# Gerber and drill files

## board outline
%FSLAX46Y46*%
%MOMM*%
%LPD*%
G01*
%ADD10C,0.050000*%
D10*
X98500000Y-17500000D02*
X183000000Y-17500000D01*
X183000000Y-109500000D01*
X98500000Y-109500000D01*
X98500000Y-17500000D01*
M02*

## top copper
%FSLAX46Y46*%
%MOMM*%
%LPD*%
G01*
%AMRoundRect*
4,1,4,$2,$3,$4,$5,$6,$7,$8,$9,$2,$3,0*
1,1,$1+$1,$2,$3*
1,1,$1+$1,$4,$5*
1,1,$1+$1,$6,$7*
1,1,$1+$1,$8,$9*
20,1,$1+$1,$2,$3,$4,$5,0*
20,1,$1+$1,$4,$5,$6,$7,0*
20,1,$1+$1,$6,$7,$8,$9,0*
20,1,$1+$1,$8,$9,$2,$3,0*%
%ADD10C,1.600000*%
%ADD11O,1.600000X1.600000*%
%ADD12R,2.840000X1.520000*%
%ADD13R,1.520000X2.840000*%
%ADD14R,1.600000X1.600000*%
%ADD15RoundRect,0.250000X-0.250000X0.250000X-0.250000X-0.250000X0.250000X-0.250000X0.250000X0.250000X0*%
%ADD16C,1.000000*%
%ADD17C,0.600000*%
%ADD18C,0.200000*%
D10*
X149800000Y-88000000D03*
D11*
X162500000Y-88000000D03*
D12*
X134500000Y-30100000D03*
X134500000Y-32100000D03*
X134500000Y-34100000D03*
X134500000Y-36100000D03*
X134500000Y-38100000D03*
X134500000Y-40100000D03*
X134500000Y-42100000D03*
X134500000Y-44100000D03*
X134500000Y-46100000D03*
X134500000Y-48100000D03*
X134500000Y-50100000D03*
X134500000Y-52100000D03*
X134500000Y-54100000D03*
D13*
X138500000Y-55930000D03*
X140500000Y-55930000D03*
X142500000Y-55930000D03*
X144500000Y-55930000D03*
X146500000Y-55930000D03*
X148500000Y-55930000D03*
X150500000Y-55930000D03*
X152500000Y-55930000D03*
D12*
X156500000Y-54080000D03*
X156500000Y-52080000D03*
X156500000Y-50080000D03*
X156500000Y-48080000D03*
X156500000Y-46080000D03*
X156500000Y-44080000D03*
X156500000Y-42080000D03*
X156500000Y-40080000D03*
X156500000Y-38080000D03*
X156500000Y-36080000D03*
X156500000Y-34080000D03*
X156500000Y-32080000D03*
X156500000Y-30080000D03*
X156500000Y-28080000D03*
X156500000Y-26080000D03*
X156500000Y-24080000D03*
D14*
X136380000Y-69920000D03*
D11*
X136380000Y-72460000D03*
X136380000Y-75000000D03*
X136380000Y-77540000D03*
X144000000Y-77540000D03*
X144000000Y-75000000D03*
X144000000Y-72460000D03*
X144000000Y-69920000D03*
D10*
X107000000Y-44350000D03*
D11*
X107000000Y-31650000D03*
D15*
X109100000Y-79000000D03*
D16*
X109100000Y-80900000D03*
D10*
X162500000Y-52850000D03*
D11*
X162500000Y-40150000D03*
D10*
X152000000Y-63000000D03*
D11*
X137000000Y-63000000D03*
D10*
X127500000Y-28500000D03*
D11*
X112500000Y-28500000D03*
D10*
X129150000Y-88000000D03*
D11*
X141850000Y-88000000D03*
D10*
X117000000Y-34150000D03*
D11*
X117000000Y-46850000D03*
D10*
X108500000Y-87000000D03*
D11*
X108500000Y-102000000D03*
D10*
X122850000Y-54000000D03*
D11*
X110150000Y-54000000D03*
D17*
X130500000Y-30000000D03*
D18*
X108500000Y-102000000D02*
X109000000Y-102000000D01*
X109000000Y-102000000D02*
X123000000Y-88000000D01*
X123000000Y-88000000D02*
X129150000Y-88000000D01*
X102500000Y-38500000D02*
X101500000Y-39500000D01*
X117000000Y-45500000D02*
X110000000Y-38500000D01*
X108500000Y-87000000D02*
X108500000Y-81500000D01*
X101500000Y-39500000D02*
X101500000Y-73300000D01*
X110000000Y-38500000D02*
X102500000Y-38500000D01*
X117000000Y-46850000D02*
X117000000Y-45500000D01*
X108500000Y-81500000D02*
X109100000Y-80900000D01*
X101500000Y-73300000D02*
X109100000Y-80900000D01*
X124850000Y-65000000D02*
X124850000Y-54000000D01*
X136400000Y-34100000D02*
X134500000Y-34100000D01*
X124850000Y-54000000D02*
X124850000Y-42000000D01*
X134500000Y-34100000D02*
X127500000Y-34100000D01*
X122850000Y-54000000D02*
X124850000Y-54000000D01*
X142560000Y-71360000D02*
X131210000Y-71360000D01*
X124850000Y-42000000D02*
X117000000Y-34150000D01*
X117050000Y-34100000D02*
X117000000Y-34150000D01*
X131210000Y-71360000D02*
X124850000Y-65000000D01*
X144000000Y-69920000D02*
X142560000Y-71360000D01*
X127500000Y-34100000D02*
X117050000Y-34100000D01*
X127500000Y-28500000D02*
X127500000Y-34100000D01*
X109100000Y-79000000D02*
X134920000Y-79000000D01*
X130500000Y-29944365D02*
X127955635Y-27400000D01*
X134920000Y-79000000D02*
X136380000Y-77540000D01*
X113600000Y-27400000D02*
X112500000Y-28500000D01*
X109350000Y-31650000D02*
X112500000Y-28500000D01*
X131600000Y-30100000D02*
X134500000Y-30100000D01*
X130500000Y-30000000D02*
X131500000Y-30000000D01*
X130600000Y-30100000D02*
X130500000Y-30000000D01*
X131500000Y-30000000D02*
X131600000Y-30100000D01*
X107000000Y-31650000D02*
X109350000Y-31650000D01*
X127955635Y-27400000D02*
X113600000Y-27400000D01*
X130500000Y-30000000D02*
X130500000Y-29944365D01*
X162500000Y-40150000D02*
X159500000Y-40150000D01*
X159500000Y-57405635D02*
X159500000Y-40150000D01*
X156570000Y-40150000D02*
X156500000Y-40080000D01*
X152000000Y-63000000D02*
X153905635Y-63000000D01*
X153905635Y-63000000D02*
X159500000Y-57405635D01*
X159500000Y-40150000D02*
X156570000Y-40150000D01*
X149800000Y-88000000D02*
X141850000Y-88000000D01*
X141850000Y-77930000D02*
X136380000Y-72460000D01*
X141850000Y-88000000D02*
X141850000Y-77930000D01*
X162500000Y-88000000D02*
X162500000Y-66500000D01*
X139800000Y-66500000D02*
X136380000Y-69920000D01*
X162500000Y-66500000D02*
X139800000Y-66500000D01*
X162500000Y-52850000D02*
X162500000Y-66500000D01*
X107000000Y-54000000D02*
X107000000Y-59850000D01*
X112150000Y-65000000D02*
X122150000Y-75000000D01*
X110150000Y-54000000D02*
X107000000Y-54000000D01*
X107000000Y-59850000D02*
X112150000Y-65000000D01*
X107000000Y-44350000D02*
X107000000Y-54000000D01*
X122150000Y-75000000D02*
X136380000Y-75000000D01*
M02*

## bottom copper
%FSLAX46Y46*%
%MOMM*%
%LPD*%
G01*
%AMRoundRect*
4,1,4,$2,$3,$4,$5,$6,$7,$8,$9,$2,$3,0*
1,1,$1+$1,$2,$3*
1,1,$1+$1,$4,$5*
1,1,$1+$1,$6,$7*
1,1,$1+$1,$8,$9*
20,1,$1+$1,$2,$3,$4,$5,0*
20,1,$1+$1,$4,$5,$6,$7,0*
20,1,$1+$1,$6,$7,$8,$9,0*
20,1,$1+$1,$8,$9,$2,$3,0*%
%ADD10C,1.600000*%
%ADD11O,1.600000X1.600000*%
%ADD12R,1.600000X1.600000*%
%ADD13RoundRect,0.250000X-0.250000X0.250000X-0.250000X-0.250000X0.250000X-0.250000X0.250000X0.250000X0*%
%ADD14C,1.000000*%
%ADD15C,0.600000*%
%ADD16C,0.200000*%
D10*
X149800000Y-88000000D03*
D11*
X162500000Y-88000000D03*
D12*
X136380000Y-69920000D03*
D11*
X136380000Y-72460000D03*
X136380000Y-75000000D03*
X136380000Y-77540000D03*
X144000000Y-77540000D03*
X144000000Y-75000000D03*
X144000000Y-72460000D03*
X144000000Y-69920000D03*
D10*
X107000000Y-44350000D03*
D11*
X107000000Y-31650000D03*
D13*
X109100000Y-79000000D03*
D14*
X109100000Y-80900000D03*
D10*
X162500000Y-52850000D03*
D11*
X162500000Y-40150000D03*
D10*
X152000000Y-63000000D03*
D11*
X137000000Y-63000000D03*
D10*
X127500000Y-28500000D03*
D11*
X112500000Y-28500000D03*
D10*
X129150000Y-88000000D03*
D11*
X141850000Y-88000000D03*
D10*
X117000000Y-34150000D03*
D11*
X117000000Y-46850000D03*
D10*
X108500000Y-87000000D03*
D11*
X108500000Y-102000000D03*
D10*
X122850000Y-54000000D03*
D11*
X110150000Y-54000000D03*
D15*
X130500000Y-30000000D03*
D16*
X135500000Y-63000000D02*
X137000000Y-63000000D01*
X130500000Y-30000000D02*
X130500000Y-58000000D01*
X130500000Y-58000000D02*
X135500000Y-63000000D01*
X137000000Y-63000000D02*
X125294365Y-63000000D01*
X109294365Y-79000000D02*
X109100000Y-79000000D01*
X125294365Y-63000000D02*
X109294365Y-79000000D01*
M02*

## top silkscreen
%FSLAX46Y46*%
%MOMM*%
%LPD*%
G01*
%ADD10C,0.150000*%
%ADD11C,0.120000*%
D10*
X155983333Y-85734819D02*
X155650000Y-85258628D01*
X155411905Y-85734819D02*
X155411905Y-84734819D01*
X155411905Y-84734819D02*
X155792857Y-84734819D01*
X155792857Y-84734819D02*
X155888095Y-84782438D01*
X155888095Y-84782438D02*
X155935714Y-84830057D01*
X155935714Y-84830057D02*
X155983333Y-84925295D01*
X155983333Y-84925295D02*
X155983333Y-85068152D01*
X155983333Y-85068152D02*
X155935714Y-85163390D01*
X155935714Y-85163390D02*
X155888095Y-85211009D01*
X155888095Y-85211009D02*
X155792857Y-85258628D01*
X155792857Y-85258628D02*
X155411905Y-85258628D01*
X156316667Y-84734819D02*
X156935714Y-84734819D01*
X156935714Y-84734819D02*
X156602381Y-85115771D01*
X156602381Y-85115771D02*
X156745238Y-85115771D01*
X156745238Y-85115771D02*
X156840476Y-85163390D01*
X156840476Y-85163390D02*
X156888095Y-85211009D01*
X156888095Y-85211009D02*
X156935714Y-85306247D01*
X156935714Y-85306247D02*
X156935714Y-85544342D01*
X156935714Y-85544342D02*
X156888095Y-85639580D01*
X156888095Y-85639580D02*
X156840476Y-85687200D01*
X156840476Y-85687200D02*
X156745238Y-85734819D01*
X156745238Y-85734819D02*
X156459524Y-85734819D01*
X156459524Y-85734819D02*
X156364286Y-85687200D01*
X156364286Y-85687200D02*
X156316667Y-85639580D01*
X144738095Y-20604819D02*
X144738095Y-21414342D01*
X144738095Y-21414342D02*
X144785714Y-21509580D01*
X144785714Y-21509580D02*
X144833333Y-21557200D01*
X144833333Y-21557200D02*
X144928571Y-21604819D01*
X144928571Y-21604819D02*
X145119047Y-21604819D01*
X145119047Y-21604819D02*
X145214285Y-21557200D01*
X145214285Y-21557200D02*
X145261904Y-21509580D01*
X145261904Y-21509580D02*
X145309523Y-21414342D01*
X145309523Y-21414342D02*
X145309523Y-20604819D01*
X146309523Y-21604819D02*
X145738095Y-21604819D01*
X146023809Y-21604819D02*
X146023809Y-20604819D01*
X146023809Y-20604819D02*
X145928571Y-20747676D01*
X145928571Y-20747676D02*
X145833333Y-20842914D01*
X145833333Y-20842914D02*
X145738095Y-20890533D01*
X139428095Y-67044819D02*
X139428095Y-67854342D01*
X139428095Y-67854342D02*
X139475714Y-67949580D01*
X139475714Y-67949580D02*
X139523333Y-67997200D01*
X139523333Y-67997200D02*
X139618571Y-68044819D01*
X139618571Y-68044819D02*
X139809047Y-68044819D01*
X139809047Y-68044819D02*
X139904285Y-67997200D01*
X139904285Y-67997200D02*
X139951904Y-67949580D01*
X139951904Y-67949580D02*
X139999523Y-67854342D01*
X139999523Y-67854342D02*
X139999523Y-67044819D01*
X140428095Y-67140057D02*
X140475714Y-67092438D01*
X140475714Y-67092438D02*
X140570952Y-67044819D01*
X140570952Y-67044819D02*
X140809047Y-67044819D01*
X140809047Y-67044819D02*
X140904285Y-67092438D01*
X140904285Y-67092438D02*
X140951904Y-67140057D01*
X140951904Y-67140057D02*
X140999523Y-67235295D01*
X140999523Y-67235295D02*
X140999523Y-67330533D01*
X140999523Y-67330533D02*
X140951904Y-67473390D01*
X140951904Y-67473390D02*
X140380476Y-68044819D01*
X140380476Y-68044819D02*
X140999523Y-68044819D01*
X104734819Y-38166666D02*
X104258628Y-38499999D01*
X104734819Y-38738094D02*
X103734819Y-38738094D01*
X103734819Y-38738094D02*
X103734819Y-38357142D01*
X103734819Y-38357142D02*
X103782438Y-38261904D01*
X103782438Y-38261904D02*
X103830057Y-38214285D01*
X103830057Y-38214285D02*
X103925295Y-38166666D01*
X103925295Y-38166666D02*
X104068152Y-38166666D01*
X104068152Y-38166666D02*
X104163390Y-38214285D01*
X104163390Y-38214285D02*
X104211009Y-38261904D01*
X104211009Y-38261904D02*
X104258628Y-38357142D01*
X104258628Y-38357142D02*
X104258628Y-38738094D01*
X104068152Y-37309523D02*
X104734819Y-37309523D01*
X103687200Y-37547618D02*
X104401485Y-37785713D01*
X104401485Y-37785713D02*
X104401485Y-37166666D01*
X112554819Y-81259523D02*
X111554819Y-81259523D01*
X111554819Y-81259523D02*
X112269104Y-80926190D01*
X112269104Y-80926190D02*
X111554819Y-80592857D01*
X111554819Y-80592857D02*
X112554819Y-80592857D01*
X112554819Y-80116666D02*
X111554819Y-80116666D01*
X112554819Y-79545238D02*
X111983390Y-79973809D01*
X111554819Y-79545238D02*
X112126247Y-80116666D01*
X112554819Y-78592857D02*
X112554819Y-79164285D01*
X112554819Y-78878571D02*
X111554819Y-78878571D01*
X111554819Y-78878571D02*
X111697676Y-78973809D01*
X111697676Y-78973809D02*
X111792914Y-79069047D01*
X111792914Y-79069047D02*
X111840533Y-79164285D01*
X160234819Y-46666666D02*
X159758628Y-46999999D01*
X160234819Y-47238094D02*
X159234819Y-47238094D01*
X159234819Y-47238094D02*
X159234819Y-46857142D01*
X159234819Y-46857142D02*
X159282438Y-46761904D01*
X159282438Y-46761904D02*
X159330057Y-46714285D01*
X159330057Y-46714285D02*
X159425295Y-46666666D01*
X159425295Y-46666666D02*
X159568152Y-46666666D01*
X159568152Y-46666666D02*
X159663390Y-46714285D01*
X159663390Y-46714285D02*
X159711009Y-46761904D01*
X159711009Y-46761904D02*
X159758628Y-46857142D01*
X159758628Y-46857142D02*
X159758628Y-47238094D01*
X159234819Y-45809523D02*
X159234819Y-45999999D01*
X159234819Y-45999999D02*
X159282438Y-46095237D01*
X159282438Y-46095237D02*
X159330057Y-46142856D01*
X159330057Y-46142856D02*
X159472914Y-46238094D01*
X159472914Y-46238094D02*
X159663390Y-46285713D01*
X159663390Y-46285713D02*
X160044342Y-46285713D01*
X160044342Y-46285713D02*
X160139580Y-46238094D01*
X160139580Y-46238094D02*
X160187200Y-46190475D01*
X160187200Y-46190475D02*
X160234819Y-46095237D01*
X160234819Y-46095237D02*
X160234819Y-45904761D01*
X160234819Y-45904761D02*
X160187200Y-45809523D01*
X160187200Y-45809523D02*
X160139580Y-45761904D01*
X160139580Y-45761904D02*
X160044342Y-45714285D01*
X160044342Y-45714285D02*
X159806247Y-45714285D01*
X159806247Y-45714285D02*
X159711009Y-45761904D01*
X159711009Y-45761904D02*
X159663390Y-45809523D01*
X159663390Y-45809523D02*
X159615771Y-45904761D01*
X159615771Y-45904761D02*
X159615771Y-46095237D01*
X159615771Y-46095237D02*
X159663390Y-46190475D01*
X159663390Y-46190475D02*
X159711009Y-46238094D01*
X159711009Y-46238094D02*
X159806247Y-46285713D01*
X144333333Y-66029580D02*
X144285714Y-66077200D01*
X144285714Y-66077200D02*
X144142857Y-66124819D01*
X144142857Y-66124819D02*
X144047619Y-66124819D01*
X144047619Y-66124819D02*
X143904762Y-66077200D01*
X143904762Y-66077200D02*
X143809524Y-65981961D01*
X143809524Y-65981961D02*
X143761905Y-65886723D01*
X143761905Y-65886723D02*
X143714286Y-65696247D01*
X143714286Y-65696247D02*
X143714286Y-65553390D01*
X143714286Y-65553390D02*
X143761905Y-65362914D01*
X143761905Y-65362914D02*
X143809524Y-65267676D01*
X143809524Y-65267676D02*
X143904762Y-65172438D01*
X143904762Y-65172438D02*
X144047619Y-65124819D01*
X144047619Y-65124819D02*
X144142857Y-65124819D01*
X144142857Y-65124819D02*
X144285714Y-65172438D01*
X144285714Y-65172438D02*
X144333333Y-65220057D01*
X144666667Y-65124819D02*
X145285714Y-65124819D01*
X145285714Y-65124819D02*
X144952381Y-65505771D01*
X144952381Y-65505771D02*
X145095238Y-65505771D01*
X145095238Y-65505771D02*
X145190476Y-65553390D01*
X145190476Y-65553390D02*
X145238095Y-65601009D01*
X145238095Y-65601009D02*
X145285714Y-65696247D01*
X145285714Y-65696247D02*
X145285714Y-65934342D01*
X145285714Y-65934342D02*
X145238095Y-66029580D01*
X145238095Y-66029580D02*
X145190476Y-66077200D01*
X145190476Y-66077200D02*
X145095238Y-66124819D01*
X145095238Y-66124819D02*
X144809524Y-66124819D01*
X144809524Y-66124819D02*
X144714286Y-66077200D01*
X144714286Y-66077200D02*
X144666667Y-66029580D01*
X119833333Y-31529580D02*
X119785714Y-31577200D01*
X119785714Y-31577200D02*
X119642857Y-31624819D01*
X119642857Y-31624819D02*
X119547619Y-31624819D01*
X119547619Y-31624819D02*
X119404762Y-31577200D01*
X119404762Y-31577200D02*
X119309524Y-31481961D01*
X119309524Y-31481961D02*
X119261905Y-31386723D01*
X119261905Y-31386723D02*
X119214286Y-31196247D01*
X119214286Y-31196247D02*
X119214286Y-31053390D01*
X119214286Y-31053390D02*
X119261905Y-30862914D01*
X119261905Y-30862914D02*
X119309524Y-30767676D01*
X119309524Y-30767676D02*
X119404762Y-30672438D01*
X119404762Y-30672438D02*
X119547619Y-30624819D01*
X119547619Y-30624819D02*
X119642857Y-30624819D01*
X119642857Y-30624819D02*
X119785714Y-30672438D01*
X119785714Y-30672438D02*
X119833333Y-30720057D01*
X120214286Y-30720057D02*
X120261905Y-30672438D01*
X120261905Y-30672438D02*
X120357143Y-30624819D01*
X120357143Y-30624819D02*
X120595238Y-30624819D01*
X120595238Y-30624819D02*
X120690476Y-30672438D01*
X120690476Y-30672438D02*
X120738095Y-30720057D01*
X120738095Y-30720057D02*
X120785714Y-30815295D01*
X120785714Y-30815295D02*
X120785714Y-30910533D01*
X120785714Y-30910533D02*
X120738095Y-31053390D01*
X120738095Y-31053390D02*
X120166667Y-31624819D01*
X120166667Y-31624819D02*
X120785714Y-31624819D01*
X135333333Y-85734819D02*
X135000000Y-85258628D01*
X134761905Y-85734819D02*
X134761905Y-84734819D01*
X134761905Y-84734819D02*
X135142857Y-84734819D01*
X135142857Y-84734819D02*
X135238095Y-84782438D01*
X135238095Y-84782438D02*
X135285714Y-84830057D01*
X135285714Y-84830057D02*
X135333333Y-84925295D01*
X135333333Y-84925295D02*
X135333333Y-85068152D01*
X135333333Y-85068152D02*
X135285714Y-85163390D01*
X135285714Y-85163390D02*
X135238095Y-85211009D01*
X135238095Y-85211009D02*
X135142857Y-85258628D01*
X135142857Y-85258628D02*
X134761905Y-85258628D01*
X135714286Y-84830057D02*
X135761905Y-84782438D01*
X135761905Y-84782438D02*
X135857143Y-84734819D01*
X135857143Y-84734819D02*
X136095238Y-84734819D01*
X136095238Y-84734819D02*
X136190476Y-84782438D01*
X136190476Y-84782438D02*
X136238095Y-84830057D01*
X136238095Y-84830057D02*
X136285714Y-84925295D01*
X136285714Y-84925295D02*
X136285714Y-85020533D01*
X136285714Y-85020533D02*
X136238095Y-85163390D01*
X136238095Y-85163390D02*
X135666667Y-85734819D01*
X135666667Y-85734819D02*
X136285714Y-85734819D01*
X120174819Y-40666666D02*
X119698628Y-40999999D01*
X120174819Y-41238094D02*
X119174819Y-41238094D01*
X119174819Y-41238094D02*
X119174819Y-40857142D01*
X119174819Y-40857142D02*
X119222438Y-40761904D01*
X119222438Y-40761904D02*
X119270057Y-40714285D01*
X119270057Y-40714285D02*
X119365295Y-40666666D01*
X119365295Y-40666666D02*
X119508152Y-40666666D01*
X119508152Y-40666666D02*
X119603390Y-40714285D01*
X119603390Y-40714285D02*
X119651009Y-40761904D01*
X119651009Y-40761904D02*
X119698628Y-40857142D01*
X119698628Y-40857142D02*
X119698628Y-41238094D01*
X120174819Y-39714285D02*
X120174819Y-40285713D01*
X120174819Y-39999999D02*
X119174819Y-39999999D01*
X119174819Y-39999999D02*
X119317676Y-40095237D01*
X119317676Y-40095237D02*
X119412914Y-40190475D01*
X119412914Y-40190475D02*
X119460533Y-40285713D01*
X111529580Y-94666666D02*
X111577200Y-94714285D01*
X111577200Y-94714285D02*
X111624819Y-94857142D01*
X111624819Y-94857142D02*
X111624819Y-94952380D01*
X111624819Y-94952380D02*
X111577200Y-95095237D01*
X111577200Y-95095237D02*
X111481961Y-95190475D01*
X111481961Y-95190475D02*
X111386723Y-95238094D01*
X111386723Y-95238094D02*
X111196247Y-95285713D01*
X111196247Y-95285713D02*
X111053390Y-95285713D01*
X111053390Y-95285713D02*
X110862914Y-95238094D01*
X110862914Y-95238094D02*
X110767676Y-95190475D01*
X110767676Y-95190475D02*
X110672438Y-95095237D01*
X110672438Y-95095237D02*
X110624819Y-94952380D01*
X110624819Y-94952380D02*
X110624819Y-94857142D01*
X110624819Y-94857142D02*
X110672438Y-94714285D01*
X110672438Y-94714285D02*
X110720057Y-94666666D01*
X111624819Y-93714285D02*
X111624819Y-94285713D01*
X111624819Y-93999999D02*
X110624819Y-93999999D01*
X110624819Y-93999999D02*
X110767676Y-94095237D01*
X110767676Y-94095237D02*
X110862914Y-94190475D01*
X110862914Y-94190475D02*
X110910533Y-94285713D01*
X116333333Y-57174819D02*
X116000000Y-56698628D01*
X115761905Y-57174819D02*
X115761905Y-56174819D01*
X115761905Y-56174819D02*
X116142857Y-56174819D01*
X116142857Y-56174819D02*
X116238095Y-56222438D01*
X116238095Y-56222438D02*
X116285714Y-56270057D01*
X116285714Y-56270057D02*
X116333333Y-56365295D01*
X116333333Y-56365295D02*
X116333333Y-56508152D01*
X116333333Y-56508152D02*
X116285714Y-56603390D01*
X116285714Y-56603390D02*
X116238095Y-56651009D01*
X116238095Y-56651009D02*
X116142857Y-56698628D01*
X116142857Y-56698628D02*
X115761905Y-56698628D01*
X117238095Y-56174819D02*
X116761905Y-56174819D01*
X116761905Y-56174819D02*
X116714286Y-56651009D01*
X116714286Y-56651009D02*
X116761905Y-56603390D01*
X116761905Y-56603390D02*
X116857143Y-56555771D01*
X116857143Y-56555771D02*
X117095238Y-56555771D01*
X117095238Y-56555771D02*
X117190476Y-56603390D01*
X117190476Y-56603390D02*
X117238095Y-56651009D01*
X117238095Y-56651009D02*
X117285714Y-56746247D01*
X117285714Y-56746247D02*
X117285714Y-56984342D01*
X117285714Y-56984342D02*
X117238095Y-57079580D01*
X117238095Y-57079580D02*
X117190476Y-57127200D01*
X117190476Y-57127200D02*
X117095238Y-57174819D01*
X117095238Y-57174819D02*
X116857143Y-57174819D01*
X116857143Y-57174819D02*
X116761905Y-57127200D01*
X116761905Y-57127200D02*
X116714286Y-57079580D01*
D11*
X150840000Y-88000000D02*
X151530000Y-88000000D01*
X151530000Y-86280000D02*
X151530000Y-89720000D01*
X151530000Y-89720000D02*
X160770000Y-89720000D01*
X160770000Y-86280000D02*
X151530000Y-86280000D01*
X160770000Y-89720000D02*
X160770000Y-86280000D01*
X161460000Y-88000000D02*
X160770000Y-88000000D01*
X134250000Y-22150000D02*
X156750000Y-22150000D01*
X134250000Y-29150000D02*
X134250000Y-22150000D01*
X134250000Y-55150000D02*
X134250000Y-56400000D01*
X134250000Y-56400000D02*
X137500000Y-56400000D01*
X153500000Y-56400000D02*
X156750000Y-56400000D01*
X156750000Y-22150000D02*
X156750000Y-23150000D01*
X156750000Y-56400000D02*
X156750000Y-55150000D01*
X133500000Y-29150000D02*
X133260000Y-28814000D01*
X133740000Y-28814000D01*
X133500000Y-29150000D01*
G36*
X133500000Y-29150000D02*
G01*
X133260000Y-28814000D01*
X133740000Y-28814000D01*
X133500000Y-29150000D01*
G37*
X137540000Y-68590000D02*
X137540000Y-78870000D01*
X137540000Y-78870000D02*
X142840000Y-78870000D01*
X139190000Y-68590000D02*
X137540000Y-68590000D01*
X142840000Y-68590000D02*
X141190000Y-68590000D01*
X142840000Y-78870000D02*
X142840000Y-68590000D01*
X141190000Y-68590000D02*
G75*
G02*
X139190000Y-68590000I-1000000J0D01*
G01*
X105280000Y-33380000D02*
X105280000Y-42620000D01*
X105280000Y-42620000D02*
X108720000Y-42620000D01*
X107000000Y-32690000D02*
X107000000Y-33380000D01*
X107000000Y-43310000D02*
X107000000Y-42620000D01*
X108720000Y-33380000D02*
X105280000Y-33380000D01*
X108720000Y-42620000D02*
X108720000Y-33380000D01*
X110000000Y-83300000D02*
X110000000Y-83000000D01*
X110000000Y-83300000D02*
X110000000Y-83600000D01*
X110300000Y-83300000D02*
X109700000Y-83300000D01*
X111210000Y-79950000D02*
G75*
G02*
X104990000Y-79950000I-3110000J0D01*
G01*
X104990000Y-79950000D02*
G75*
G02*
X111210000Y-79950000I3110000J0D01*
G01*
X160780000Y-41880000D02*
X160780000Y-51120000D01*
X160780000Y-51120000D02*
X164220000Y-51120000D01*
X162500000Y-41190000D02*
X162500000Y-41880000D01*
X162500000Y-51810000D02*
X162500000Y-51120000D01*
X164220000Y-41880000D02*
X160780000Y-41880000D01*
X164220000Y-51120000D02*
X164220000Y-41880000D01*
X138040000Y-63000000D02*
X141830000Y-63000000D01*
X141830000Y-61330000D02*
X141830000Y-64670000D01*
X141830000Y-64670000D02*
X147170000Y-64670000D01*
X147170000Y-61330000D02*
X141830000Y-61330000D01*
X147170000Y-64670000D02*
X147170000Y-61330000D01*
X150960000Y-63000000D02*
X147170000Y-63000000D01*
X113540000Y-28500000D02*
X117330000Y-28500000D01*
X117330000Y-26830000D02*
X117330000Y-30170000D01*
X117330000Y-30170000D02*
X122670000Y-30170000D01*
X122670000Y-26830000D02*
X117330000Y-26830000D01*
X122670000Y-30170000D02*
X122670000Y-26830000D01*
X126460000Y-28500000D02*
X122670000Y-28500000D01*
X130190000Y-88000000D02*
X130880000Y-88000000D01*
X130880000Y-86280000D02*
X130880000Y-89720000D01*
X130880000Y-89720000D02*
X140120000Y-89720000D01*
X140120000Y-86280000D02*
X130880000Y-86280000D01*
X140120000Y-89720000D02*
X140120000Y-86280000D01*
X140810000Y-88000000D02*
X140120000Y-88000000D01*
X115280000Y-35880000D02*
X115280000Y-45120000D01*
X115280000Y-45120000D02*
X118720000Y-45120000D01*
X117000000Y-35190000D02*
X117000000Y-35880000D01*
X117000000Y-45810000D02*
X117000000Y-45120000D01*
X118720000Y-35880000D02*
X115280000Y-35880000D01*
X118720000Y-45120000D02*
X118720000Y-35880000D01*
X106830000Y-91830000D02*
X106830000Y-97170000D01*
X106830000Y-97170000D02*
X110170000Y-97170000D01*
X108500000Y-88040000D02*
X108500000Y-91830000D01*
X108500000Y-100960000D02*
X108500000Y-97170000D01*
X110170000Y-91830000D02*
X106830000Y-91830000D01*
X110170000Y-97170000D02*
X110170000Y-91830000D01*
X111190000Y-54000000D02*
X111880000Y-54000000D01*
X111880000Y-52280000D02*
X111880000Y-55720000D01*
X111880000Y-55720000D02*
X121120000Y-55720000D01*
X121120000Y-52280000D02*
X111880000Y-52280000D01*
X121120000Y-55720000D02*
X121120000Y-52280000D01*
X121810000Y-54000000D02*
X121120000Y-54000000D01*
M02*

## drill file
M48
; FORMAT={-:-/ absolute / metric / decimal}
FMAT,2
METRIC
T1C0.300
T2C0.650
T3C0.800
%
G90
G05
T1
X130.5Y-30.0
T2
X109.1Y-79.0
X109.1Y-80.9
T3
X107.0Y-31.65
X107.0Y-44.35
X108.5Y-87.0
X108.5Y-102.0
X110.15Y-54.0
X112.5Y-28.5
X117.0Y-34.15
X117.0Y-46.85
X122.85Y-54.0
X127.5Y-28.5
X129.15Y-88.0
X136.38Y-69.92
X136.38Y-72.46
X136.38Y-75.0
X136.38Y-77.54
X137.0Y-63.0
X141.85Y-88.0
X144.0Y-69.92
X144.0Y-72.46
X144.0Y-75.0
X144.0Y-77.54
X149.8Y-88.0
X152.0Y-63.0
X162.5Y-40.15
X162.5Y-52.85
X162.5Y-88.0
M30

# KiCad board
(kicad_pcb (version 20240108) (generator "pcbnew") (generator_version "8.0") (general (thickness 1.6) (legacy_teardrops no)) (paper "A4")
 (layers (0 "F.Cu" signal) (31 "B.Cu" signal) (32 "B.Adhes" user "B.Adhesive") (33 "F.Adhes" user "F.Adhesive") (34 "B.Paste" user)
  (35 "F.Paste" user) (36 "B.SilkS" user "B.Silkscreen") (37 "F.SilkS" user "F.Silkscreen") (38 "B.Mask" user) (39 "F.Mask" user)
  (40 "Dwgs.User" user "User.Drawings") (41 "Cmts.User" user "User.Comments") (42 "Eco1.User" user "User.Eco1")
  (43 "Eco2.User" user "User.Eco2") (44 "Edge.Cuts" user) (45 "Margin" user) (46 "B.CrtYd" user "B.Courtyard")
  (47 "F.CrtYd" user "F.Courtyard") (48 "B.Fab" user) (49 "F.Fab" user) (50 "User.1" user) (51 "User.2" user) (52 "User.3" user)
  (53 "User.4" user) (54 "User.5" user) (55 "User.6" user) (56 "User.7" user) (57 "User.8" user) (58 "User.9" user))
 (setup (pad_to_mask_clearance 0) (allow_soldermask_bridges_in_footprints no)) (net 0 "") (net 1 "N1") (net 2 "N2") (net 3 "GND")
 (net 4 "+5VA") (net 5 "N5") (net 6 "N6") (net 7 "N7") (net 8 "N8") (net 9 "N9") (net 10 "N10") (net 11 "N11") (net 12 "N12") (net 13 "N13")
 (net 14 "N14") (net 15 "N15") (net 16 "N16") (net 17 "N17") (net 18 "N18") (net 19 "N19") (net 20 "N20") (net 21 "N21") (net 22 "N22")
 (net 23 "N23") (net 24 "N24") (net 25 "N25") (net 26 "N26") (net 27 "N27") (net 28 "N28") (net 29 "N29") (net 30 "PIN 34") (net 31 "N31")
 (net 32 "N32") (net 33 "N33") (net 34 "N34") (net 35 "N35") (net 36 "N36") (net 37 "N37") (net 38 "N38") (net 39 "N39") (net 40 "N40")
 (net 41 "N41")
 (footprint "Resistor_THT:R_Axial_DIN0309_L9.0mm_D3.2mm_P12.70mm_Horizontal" (layer "F.Cu") (at 149.8 88)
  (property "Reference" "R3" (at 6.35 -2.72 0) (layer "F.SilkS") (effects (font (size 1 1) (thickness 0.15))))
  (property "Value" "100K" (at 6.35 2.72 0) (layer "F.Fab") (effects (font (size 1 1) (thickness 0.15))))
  (fp_line (start 1.04 0) (end 1.73 0) (stroke (width 0.12) (type solid)) (layer "F.SilkS"))
  (fp_line (start 1.73 -1.72) (end 1.73 1.72) (stroke (width 0.12) (type solid)) (layer "F.SilkS"))
  (fp_line (start 1.73 1.72) (end 10.97 1.72) (stroke (width 0.12) (type solid)) (layer "F.SilkS"))
  (fp_line (start 10.97 -1.72) (end 1.73 -1.72) (stroke (width 0.12) (type solid)) (layer "F.SilkS"))
  (fp_line (start 10.97 1.72) (end 10.97 -1.72) (stroke (width 0.12) (type solid)) (layer "F.SilkS"))
  (fp_line (start 11.66 0) (end 10.97 0) (stroke (width 0.12) (type solid)) (layer "F.SilkS"))
  (pad "1" thru_hole circle (at 0 0) (size 1.6 1.6) (drill 0.8) (layers "*.Cu" "*.Mask") (remove_unused_layers no) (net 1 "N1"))
  (pad "2" thru_hole oval (at 12.7 0) (size 1.6 1.6) (drill 0.8) (layers "*.Cu" "*.Mask") (remove_unused_layers no) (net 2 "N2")))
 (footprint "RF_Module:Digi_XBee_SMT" (layer "F.Cu") (at 145.5 40)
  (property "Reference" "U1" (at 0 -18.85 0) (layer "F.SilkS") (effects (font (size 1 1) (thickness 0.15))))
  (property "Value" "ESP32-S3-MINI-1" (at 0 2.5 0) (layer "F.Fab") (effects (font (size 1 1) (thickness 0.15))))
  (fp_line (start -11.25 -17.85) (end 11.25 -17.85) (stroke (width 0.12) (type solid)) (layer "F.SilkS"))
  (fp_line (start -11.25 -10.85) (end -11.25 -17.85) (stroke (width 0.12) (type solid)) (layer "F.SilkS"))
  (fp_line (start -11.25 15.15) (end -11.25 16.4) (stroke (width 0.12) (type solid)) (layer "F.SilkS"))
  (fp_line (start -11.25 16.4) (end -8 16.4) (stroke (width 0.12) (type solid)) (layer "F.SilkS"))
  (fp_line (start 8 16.4) (end 11.25 16.4) (stroke (width 0.12) (type solid)) (layer "F.SilkS"))
  (fp_line (start 11.25 -17.85) (end 11.25 -16.85) (stroke (width 0.12) (type solid)) (layer "F.SilkS"))
  (fp_line (start 11.25 16.4) (end 11.25 15.15) (stroke (width 0.12) (type solid)) (layer "F.SilkS"))
  (fp_poly
   (pts (xy -12 -10.85) (xy -12.24 -11.186) (xy -11.76 -11.186) (xy -12 -10.85)) (stroke (width 0.12) (type solid)) (fill solid)
   (layer "F.SilkS"))
  (pad "1" smd rect (at -11 -9.9) (size 2.84 1.52) (layers "F.Cu" "F.Paste" "F.Mask") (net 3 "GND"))
  (pad "2" smd rect (at -11 -7.9) (size 2.84 1.52) (layers "F.Cu" "F.Paste" "F.Mask") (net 3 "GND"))
  (pad "3" smd rect (at -11 -5.9) (size 2.84 1.52) (layers "F.Cu" "F.Paste" "F.Mask") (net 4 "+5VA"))
  (pad "4" smd rect (at -11 -3.9) (size 2.84 1.52) (layers "F.Cu" "F.Paste" "F.Mask") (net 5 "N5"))
  (pad "5" smd rect (at -11 -1.9) (size 2.84 1.52) (layers "F.Cu" "F.Paste" "F.Mask") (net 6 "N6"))
  (pad "6" smd rect (at -11 0.1) (size 2.84 1.52) (layers "F.Cu" "F.Paste" "F.Mask") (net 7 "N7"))
  (pad "7" smd rect (at -11 2.1) (size 2.84 1.52) (layers "F.Cu" "F.Paste" "F.Mask") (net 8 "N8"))
  (pad "8" smd rect (at -11 4.1) (size 2.84 1.52) (layers "F.Cu" "F.Paste" "F.Mask") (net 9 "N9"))
  (pad "9" smd rect (at -11 6.1) (size 2.84 1.52) (layers "F.Cu" "F.Paste" "F.Mask") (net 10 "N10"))
  (pad "10" smd rect (at -11 8.1) (size 2.84 1.52) (layers "F.Cu" "F.Paste" "F.Mask") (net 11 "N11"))
  (pad "11" smd rect (at -11 10.1) (size 2.84 1.52) (layers "F.Cu" "F.Paste" "F.Mask") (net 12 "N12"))
  (pad "12" smd rect (at -11 12.1) (size 2.84 1.52) (layers "F.Cu" "F.Paste" "F.Mask") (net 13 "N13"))
  (pad "13" smd rect (at -11 14.1) (size 2.84 1.52) (layers "F.Cu" "F.Paste" "F.Mask") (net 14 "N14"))
  (pad "14" smd rect (at -7 15.93 90) (size 2.84 1.52) (layers "F.Cu" "F.Paste" "F.Mask") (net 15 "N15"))
  (pad "15" smd rect (at -5 15.93 90) (size 2.84 1.52) (layers "F.Cu" "F.Paste" "F.Mask") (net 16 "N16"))
  (pad "16" smd rect (at -3 15.93 90) (size 2.84 1.52) (layers "F.Cu" "F.Paste" "F.Mask") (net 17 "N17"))
  (pad "17" smd rect (at -1 15.93 90) (size 2.84 1.52) (layers "F.Cu" "F.Paste" "F.Mask") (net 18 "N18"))
  (pad "18" smd rect (at 1 15.93 90) (size 2.84 1.52) (layers "F.Cu" "F.Paste" "F.Mask") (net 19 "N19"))
  (pad "19" smd rect (at 3 15.93 90) (size 2.84 1.52) (layers "F.Cu" "F.Paste" "F.Mask") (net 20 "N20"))
  (pad "20" smd rect (at 5 15.93 90) (size 2.84 1.52) (layers "F.Cu" "F.Paste" "F.Mask") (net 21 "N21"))
  (pad "21" smd rect (at 7 15.93 90) (size 2.84 1.52) (layers "F.Cu" "F.Paste" "F.Mask") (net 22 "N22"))
  (pad "22" smd rect (at 11 14.08) (size 2.84 1.52) (layers "F.Cu" "F.Paste" "F.Mask") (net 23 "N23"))
  (pad "23" smd rect (at 11 12.08) (size 2.84 1.52) (layers "F.Cu" "F.Paste" "F.Mask") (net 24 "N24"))
  (pad "24" smd rect (at 11 10.08) (size 2.84 1.52) (layers "F.Cu" "F.Paste" "F.Mask") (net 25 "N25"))
  (pad "25" smd rect (at 11 8.08) (size 2.84 1.52) (layers "F.Cu" "F.Paste" "F.Mask") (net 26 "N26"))
  (pad "26" smd rect (at 11 6.08) (size 2.84 1.52) (layers "F.Cu" "F.Paste" "F.Mask") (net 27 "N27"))
  (pad "27" smd rect (at 11 4.08) (size 2.84 1.52) (layers "F.Cu" "F.Paste" "F.Mask") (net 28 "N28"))
  (pad "28" smd rect (at 11 2.08) (size 2.84 1.52) (layers "F.Cu" "F.Paste" "F.Mask") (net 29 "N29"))
  (pad "29" smd rect (at 11 0.08) (size 2.84 1.52) (layers "F.Cu" "F.Paste" "F.Mask") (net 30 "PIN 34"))
  (pad "30" smd rect (at 11 -1.92) (size 2.84 1.52) (layers "F.Cu" "F.Paste" "F.Mask") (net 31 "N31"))
  (pad "31" smd rect (at 11 -3.92) (size 2.84 1.52) (layers "F.Cu" "F.Paste" "F.Mask") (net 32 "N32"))
  (pad "32" smd rect (at 11 -5.92) (size 2.84 1.52) (layers "F.Cu" "F.Paste" "F.Mask") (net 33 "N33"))
  (pad "33" smd rect (at 11 -7.92) (size 2.84 1.52) (layers "F.Cu" "F.Paste" "F.Mask") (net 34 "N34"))
  (pad "34" smd rect (at 11 -9.92) (size 2.84 1.52) (layers "F.Cu" "F.Paste" "F.Mask") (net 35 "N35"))
  (pad "35" smd rect (at 11 -11.92) (size 2.84 1.52) (layers "F.Cu" "F.Paste" "F.Mask") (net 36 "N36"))
  (pad "36" smd rect (at 11 -13.92) (size 2.84 1.52) (layers "F.Cu" "F.Paste" "F.Mask") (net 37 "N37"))
  (pad "37" smd rect (at 11 -15.92) (size 2.84 1.52) (layers "F.Cu" "F.Paste" "F.Mask") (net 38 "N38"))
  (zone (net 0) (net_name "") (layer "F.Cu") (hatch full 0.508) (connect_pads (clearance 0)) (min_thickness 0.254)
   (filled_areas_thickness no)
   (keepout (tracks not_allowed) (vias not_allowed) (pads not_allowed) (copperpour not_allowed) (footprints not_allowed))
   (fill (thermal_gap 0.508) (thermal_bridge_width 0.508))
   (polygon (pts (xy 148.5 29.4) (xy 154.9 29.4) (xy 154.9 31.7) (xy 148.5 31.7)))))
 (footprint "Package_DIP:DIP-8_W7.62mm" (layer "F.Cu") (at 136.38 69.92)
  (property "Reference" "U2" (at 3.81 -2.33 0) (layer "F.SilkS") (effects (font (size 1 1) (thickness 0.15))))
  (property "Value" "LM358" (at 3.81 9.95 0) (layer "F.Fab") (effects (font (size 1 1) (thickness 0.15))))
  (fp_line (start 1.16 -1.33) (end 1.16 8.95) (stroke (width 0.12) (type solid)) (layer "F.SilkS"))
  (fp_line (start 1.16 8.95) (end 6.46 8.95) (stroke (width 0.12) (type solid)) (layer "F.SilkS"))
  (fp_line (start 2.81 -1.33) (end 1.16 -1.33) (stroke (width 0.12) (type solid)) (layer "F.SilkS"))
  (fp_line (start 6.46 -1.33) (end 4.81 -1.33) (stroke (width 0.12) (type solid)) (layer "F.SilkS"))
  (fp_line (start 6.46 8.95) (end 6.46 -1.33) (stroke (width 0.12) (type solid)) (layer "F.SilkS"))
  (fp_arc (start 4.81 -1.33) (mid 3.81 -0.33) (end 2.81 -1.33) (stroke (width 0.12) (type solid)) (layer "F.SilkS"))
  (pad "1" thru_hole rect (at 0 0) (size 1.6 1.6) (drill 0.8) (layers "*.Cu" "*.Mask") (remove_unused_layers no) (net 2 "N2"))
  (pad "2" thru_hole oval (at 0 2.54) (size 1.6 1.6) (drill 0.8) (layers "*.Cu" "*.Mask") (remove_unused_layers no) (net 1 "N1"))
  (pad "3" thru_hole oval (at 0 5.08) (size 1.6 1.6) (drill 0.8) (layers "*.Cu" "*.Mask") (remove_unused_layers no) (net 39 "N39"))
  (pad "4" thru_hole oval (at 0 7.62) (size 1.6 1.6) (drill 0.8) (layers "*.Cu" "*.Mask") (remove_unused_layers no) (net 3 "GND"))
  (pad "5" thru_hole oval (at 7.62 7.62) (size 1.6 1.6) (drill 0.8) (layers "*.Cu" "*.Mask") (remove_unused_layers no))
  (pad "6" thru_hole oval (at 7.62 5.08) (size 1.6 1.6) (drill 0.8) (layers "*.Cu" "*.Mask") (remove_unused_layers no))
  (pad "7" thru_hole oval (at 7.62 2.54) (size 1.6 1.6) (drill 0.8) (layers "*.Cu" "*.Mask") (remove_unused_layers no))
  (pad "8" thru_hole oval (at 7.62 0) (size 1.6 1.6) (drill 0.8) (layers "*.Cu" "*.Mask") (remove_unused_layers no) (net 4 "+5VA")))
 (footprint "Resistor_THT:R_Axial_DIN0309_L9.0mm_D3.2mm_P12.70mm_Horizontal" (layer "F.Cu") (at 107 44.35 90)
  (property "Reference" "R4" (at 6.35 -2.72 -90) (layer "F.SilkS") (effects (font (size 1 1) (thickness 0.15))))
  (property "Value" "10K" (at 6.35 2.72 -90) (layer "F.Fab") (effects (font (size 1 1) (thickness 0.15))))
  (fp_line (start 10.97 -1.72) (end 1.73 -1.72) (stroke (width 0.12) (type solid)) (layer "F.SilkS"))
  (fp_line (start 1.73 -1.72) (end 1.73 1.72) (stroke (width 0.12) (type solid)) (layer "F.SilkS"))
  (fp_line (start 11.66 0) (end 10.97 0) (stroke (width 0.12) (type solid)) (layer "F.SilkS"))
  (fp_line (start 1.04 0) (end 1.73 0) (stroke (width 0.12) (type solid)) (layer "F.SilkS"))
  (fp_line (start 10.97 1.72) (end 10.97 -1.72) (stroke (width 0.12) (type solid)) (layer "F.SilkS"))
  (fp_line (start 1.73 1.72) (end 10.97 1.72) (stroke (width 0.12) (type solid)) (layer "F.SilkS"))
  (pad "1" thru_hole circle (at 0 0 90) (size 1.6 1.6) (drill 0.8) (layers "*.Cu" "*.Mask") (remove_unused_layers no) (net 39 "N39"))
  (pad "2" thru_hole oval (at 12.7 0 90) (size 1.6 1.6) (drill 0.8) (layers "*.Cu" "*.Mask") (remove_unused_layers no) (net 3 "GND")))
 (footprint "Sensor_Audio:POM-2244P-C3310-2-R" (layer "F.Cu") (at 109.1 79 -90)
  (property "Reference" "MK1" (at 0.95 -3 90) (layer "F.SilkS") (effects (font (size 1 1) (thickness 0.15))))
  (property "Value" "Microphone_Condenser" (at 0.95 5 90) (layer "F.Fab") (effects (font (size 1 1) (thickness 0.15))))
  (fp_line (start 4.3 -0.9) (end 4 -0.9) (stroke (width 0.12) (type default)) (layer "F.SilkS"))
  (fp_line (start 4.3 -0.9) (end 4.6 -0.9) (stroke (width 0.12) (type default)) (layer "F.SilkS"))
  (fp_line (start 4.3 -1.2) (end 4.3 -0.6) (stroke (width 0.12) (type default)) (layer "F.SilkS"))
  (fp_circle (center 0.95 1) (end 4.06 1) (stroke (width 0.12) (type default)) (fill none) (layer "F.SilkS"))
  (pad "1" thru_hole roundrect (at 0 0 270) (size 1 1) (drill 0.65) (layers "*.Cu" "*.Mask") (remove_unused_layers no)
   (roundrect_rratio 0.25) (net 3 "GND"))
  (pad "2" thru_hole circle (at 1.9 0 270) (size 1 1) (drill 0.65) (layers "*.Cu" "*.Mask") (remove_unused_layers no) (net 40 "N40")))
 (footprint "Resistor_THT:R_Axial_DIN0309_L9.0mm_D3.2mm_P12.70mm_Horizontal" (layer "F.Cu") (at 162.5 52.85 90)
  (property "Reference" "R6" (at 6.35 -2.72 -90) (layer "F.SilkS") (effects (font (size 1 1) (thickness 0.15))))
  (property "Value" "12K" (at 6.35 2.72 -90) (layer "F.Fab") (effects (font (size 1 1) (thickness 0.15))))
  (fp_line (start 10.97 -1.72) (end 1.73 -1.72) (stroke (width 0.12) (type solid)) (layer "F.SilkS"))
  (fp_line (start 1.73 -1.72) (end 1.73 1.72) (stroke (width 0.12) (type solid)) (layer "F.SilkS"))
  (fp_line (start 11.66 0) (end 10.97 0) (stroke (width 0.12) (type solid)) (layer "F.SilkS"))
  (fp_line (start 1.04 0) (end 1.73 0) (stroke (width 0.12) (type solid)) (layer "F.SilkS"))
  (fp_line (start 10.97 1.72) (end 10.97 -1.72) (stroke (width 0.12) (type solid)) (layer "F.SilkS"))
  (fp_line (start 1.73 1.72) (end 10.97 1.72) (stroke (width 0.12) (type solid)) (layer "F.SilkS"))
  (pad "1" thru_hole circle (at 0 0 90) (size 1.6 1.6) (drill 0.8) (layers "*.Cu" "*.Mask") (remove_unused_layers no) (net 2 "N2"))
  (pad "2" thru_hole oval (at 12.7 0 90) (size 1.6 1.6) (drill 0.8) (layers "*.Cu" "*.Mask") (remove_unused_layers no) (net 30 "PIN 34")))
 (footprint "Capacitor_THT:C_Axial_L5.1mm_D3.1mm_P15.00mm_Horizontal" (layer "F.Cu") (at 152 63 180)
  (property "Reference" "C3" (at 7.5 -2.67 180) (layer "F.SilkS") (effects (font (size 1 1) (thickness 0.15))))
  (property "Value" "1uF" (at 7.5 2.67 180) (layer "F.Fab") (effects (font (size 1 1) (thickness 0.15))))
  (fp_line (start 13.96 0) (end 10.17 0) (stroke (width 0.12) (type solid)) (layer "F.SilkS"))
  (fp_line (start 10.17 1.67) (end 10.17 -1.67) (stroke (width 0.12) (type solid)) (layer "F.SilkS"))
  (fp_line (start 10.17 -1.67) (end 4.83 -1.67) (stroke (width 0.12) (type solid)) (layer "F.SilkS"))
  (fp_line (start 4.83 1.67) (end 10.17 1.67) (stroke (width 0.12) (type solid)) (layer "F.SilkS"))
  (fp_line (start 4.83 -1.67) (end 4.83 1.67) (stroke (width 0.12) (type solid)) (layer "F.SilkS"))
  (fp_line (start 1.04 0) (end 4.83 0) (stroke (width 0.12) (type solid)) (layer "F.SilkS"))
  (pad "1" thru_hole circle (at 0 0 180) (size 1.6 1.6) (drill 0.8) (layers "*.Cu" "*.Mask") (remove_unused_layers no) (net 30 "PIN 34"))
  (pad "2" thru_hole oval (at 15 0 180) (size 1.6 1.6) (drill 0.8) (layers "*.Cu" "*.Mask") (remove_unused_layers no) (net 3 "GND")))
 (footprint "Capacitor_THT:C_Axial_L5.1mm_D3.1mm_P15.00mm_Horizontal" (layer "F.Cu") (at 127.5 28.5 180)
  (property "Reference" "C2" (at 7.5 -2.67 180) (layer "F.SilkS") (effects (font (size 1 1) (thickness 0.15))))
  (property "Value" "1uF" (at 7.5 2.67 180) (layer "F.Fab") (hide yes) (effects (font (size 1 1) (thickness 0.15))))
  (fp_line (start 13.96 0) (end 10.17 0) (stroke (width 0.12) (type solid)) (layer "F.SilkS"))
  (fp_line (start 10.17 1.67) (end 10.17 -1.67) (stroke (width 0.12) (type solid)) (layer "F.SilkS"))
  (fp_line (start 10.17 -1.67) (end 4.83 -1.67) (stroke (width 0.12) (type solid)) (layer "F.SilkS"))
  (fp_line (start 4.83 1.67) (end 10.17 1.67) (stroke (width 0.12) (type solid)) (layer "F.SilkS"))
  (fp_line (start 4.83 -1.67) (end 4.83 1.67) (stroke (width 0.12) (type solid)) (layer "F.SilkS"))
  (fp_line (start 1.04 0) (end 4.83 0) (stroke (width 0.12) (type solid)) (layer "F.SilkS"))
  (pad "1" thru_hole circle (at 0 0 180) (size 1.6 1.6) (drill 0.8) (layers "*.Cu" "*.Mask") (remove_unused_layers no) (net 4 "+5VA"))
  (pad "2" thru_hole oval (at 15 0 180) (size 1.6 1.6) (drill 0.8) (layers "*.Cu" "*.Mask") (remove_unused_layers no) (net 3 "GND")))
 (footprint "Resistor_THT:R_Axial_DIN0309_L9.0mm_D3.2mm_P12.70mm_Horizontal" (layer "F.Cu") (at 129.15 88)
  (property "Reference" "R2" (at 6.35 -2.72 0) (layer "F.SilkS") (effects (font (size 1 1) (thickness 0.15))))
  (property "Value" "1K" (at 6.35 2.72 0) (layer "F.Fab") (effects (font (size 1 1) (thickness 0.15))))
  (fp_line (start 1.04 0) (end 1.73 0) (stroke (width 0.12) (type solid)) (layer "F.SilkS"))
  (fp_line (start 1.73 -1.72) (end 1.73 1.72) (stroke (width 0.12) (type solid)) (layer "F.SilkS"))
  (fp_line (start 1.73 1.72) (end 10.97 1.72) (stroke (width 0.12) (type solid)) (layer "F.SilkS"))
  (fp_line (start 10.97 -1.72) (end 1.73 -1.72) (stroke (width 0.12) (type solid)) (layer "F.SilkS"))
  (fp_line (start 10.97 1.72) (end 10.97 -1.72) (stroke (width 0.12) (type solid)) (layer "F.SilkS"))
  (fp_line (start 11.66 0) (end 10.97 0) (stroke (width 0.12) (type solid)) (layer "F.SilkS"))
  (pad "1" thru_hole circle (at 0 0) (size 1.6 1.6) (drill 0.8) (layers "*.Cu" "*.Mask") (remove_unused_layers no) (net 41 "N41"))
  (pad "2" thru_hole oval (at 12.7 0) (size 1.6 1.6) (drill 0.8) (layers "*.Cu" "*.Mask") (remove_unused_layers no) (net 1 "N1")))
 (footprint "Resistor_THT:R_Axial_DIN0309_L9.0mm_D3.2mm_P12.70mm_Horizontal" (layer "F.Cu") (at 117 34.15 -90)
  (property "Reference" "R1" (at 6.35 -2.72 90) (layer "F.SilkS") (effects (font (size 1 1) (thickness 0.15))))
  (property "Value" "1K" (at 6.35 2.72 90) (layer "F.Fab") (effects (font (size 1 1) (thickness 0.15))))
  (fp_line (start 1.73 1.72) (end 10.97 1.72) (stroke (width 0.12) (type solid)) (layer "F.SilkS"))
  (fp_line (start 10.97 1.72) (end 10.97 -1.72) (stroke (width 0.12) (type solid)) (layer "F.SilkS"))
  (fp_line (start 1.04 0) (end 1.73 0) (stroke (width 0.12) (type solid)) (layer "F.SilkS"))
  (fp_line (start 11.66 0) (end 10.97 0) (stroke (width 0.12) (type solid)) (layer "F.SilkS"))
  (fp_line (start 1.73 -1.72) (end 1.73 1.72) (stroke (width 0.12) (type solid)) (layer "F.SilkS"))
  (fp_line (start 10.97 -1.72) (end 1.73 -1.72) (stroke (width 0.12) (type solid)) (layer "F.SilkS"))
  (pad "1" thru_hole circle (at 0 0 270) (size 1.6 1.6) (drill 0.8) (layers "*.Cu" "*.Mask") (remove_unused_layers no) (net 4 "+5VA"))
  (pad "2" thru_hole oval (at 12.7 0 270) (size 1.6 1.6) (drill 0.8) (layers "*.Cu" "*.Mask") (remove_unused_layers no) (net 40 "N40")))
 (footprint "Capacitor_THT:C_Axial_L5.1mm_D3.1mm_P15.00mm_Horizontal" (layer "F.Cu") (at 108.5 87 -90)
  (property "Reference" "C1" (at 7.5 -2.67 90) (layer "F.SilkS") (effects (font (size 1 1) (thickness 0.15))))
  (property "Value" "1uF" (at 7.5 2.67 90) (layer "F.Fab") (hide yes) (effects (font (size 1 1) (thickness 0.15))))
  (fp_line (start 4.83 1.67) (end 10.17 1.67) (stroke (width 0.12) (type solid)) (layer "F.SilkS"))
  (fp_line (start 10.17 1.67) (end 10.17 -1.67) (stroke (width 0.12) (type solid)) (layer "F.SilkS"))
  (fp_line (start 1.04 0) (end 4.83 0) (stroke (width 0.12) (type solid)) (layer "F.SilkS"))
  (fp_line (start 13.96 0) (end 10.17 0) (stroke (width 0.12) (type solid)) (layer "F.SilkS"))
  (fp_line (start 4.83 -1.67) (end 4.83 1.67) (stroke (width 0.12) (type solid)) (layer "F.SilkS"))
  (fp_line (start 10.17 -1.67) (end 4.83 -1.67) (stroke (width 0.12) (type solid)) (layer "F.SilkS"))
  (pad "1" thru_hole circle (at 0 0 270) (size 1.6 1.6) (drill 0.8) (layers "*.Cu" "*.Mask") (remove_unused_layers no) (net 40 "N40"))
  (pad "2" thru_hole oval (at 15 0 270) (size 1.6 1.6) (drill 0.8) (layers "*.Cu" "*.Mask") (remove_unused_layers no) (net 41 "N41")))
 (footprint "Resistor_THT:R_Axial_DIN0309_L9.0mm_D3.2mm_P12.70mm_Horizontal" (layer "F.Cu") (at 122.85 54 180)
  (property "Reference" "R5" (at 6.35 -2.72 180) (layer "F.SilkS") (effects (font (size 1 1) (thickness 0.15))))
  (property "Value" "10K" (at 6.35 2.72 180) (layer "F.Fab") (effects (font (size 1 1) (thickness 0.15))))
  (fp_line (start 11.66 0) (end 10.97 0) (stroke (width 0.12) (type solid)) (layer "F.SilkS"))
  (fp_line (start 10.97 1.72) (end 10.97 -1.72) (stroke (width 0.12) (type solid)) (layer "F.SilkS"))
  (fp_line (start 10.97 -1.72) (end 1.73 -1.72) (stroke (width 0.12) (type solid)) (layer "F.SilkS"))
  (fp_line (start 1.73 1.72) (end 10.97 1.72) (stroke (width 0.12) (type solid)) (layer "F.SilkS"))
  (fp_line (start 1.73 -1.72) (end 1.73 1.72) (stroke (width 0.12) (type solid)) (layer "F.SilkS"))
  (fp_line (start 1.04 0) (end 1.73 0) (stroke (width 0.12) (type solid)) (layer "F.SilkS"))
  (pad "1" thru_hole circle (at 0 0 180) (size 1.6 1.6) (drill 0.8) (layers "*.Cu" "*.Mask") (remove_unused_layers no) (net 4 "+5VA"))
  (pad "2" thru_hole oval (at 12.7 0 180) (size 1.6 1.6) (drill 0.8) (layers "*.Cu" "*.Mask") (remove_unused_layers no) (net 39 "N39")))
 (gr_rect (start 98.5 17.5) (end 183 109.5) (stroke (width 0.05) (type default)) (fill none) (layer "Edge.Cuts"))
 (segment (start 108.5 102) (end 109 102) (width 0.2) (layer "F.Cu") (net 41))
 (segment (start 109 102) (end 123 88) (width 0.2) (layer "F.Cu") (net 41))
 (segment (start 123 88) (end 129.15 88) (width 0.2) (layer "F.Cu") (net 41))
 (segment (start 102.5 38.5) (end 101.5 39.5) (width 0.2) (layer "F.Cu") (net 40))
 (segment (start 117 45.5) (end 110 38.5) (width 0.2) (layer "F.Cu") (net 40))
 (segment (start 108.5 87) (end 108.5 81.5) (width 0.2) (layer "F.Cu") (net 40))
 (segment (start 101.5 39.5) (end 101.5 73.3) (width 0.2) (layer "F.Cu") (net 40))
 (segment (start 110 38.5) (end 102.5 38.5) (width 0.2) (layer "F.Cu") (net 40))
 (segment (start 117 46.85) (end 117 45.5) (width 0.2) (layer "F.Cu") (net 40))
 (segment (start 108.5 81.5) (end 109.1 80.9) (width 0.2) (layer "F.Cu") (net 40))
 (segment (start 101.5 73.3) (end 109.1 80.9) (width 0.2) (layer "F.Cu") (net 40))
 (segment (start 124.85 65) (end 124.85 54) (width 0.2) (layer "F.Cu") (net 4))
 (segment (start 136.4 34.1) (end 134.5 34.1) (width 0.2) (layer "F.Cu") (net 4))
 (segment (start 124.85 54) (end 124.85 42) (width 0.2) (layer "F.Cu") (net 4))
 (segment (start 134.5 34.1) (end 127.5 34.1) (width 0.2) (layer "F.Cu") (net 4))
 (segment (start 122.85 54) (end 124.85 54) (width 0.2) (layer "F.Cu") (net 4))
 (segment (start 142.56 71.36) (end 131.21 71.36) (width 0.2) (layer "F.Cu") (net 4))
 (segment (start 124.85 42) (end 117 34.15) (width 0.2) (layer "F.Cu") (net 4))
 (segment (start 117.05 34.1) (end 117 34.15) (width 0.2) (layer "F.Cu") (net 4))
 (segment (start 131.21 71.36) (end 124.85 65) (width 0.2) (layer "F.Cu") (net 4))
 (segment (start 144 69.92) (end 142.56 71.36) (width 0.2) (layer "F.Cu") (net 4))
 (segment (start 127.5 34.1) (end 117.05 34.1) (width 0.2) (layer "F.Cu") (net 4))
 (segment (start 127.5 28.5) (end 127.5 34.1) (width 0.2) (layer "F.Cu") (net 4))
 (segment (start 109.1 79) (end 134.92 79) (width 0.2) (layer "F.Cu") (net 3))
 (segment (start 130.5 29.944365) (end 127.955635 27.4) (width 0.2) (layer "F.Cu") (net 3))
 (segment (start 134.92 79) (end 136.38 77.54) (width 0.2) (layer "F.Cu") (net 3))
 (segment (start 113.6 27.4) (end 112.5 28.5) (width 0.2) (layer "F.Cu") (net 3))
 (segment (start 109.35 31.65) (end 112.5 28.5) (width 0.2) (layer "F.Cu") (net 3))
 (segment (start 131.6 30.1) (end 134.5 30.1) (width 0.2) (layer "F.Cu") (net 3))
 (segment (start 130.5 30) (end 131.5 30) (width 0.2) (layer "F.Cu") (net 3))
 (segment (start 130.6 30.1) (end 130.5 30) (width 0.2) (layer "F.Cu") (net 3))
 (segment (start 131.5 30) (end 131.6 30.1) (width 0.2) (layer "F.Cu") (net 3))
 (segment (start 107 31.65) (end 109.35 31.65) (width 0.2) (layer "F.Cu") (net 3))
 (segment (start 127.955635 27.4) (end 113.6 27.4) (width 0.2) (layer "F.Cu") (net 3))
 (segment (start 130.5 30) (end 130.5 29.944365) (width 0.2) (layer "F.Cu") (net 3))
 (via (at 130.5 30) (size 0.6) (drill 0.3) (layers "F.Cu" "B.Cu") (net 3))
 (segment (start 135.5 63) (end 137 63) (width 0.2) (layer "B.Cu") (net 3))
 (segment (start 130.5 30) (end 130.5 58) (width 0.2) (layer "B.Cu") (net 3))
 (segment (start 130.5 58) (end 135.5 63) (width 0.2) (layer "B.Cu") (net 3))
 (segment (start 137 63) (end 125.294365 63) (width 0.2) (layer "B.Cu") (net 3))
 (segment (start 109.294365 79) (end 109.1 79) (width 0.2) (layer "B.Cu") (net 3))
 (segment (start 125.294365 63) (end 109.294365 79) (width 0.2) (layer "B.Cu") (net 3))
 (segment (start 162.5 40.15) (end 159.5 40.15) (width 0.2) (layer "F.Cu") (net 30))
 (segment (start 159.5 57.405635) (end 159.5 40.15) (width 0.2) (layer "F.Cu") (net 30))
 (segment (start 156.57 40.15) (end 156.5 40.08) (width 0.2) (layer "F.Cu") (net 30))
 (segment (start 152 63) (end 153.905635 63) (width 0.2) (layer "F.Cu") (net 30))
 (segment (start 153.905635 63) (end 159.5 57.405635) (width 0.2) (layer "F.Cu") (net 30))
 (segment (start 159.5 40.15) (end 156.57 40.15) (width 0.2) (layer "F.Cu") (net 30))
 (segment (start 149.8 88) (end 141.85 88) (width 0.2) (layer "F.Cu") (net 1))
 (segment (start 141.85 77.93) (end 136.38 72.46) (width 0.2) (layer "F.Cu") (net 1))
 (segment (start 141.85 88) (end 141.85 77.93) (width 0.2) (layer "F.Cu") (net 1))
 (segment (start 162.5 88) (end 162.5 66.5) (width 0.2) (layer "F.Cu") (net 2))
 (segment (start 139.8 66.5) (end 136.38 69.92) (width 0.2) (layer "F.Cu") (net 2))
 (segment (start 162.5 66.5) (end 139.8 66.5) (width 0.2) (layer "F.Cu") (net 2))
 (segment (start 162.5 52.85) (end 162.5 66.5) (width 0.2) (layer "F.Cu") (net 2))
 (segment (start 107 54) (end 107 59.85) (width 0.2) (layer "F.Cu") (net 39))
 (segment (start 112.15 65) (end 122.15 75) (width 0.2) (layer "F.Cu") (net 39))
 (segment (start 110.15 54) (end 107 54) (width 0.2) (layer "F.Cu") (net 39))
 (segment (start 107 59.85) (end 112.15 65) (width 0.2) (layer "F.Cu") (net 39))
 (segment (start 107 44.35) (end 107 54) (width 0.2) (layer "F.Cu") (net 39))
 (segment (start 122.15 75) (end 136.38 75) (width 0.2) (layer "F.Cu") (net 39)))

